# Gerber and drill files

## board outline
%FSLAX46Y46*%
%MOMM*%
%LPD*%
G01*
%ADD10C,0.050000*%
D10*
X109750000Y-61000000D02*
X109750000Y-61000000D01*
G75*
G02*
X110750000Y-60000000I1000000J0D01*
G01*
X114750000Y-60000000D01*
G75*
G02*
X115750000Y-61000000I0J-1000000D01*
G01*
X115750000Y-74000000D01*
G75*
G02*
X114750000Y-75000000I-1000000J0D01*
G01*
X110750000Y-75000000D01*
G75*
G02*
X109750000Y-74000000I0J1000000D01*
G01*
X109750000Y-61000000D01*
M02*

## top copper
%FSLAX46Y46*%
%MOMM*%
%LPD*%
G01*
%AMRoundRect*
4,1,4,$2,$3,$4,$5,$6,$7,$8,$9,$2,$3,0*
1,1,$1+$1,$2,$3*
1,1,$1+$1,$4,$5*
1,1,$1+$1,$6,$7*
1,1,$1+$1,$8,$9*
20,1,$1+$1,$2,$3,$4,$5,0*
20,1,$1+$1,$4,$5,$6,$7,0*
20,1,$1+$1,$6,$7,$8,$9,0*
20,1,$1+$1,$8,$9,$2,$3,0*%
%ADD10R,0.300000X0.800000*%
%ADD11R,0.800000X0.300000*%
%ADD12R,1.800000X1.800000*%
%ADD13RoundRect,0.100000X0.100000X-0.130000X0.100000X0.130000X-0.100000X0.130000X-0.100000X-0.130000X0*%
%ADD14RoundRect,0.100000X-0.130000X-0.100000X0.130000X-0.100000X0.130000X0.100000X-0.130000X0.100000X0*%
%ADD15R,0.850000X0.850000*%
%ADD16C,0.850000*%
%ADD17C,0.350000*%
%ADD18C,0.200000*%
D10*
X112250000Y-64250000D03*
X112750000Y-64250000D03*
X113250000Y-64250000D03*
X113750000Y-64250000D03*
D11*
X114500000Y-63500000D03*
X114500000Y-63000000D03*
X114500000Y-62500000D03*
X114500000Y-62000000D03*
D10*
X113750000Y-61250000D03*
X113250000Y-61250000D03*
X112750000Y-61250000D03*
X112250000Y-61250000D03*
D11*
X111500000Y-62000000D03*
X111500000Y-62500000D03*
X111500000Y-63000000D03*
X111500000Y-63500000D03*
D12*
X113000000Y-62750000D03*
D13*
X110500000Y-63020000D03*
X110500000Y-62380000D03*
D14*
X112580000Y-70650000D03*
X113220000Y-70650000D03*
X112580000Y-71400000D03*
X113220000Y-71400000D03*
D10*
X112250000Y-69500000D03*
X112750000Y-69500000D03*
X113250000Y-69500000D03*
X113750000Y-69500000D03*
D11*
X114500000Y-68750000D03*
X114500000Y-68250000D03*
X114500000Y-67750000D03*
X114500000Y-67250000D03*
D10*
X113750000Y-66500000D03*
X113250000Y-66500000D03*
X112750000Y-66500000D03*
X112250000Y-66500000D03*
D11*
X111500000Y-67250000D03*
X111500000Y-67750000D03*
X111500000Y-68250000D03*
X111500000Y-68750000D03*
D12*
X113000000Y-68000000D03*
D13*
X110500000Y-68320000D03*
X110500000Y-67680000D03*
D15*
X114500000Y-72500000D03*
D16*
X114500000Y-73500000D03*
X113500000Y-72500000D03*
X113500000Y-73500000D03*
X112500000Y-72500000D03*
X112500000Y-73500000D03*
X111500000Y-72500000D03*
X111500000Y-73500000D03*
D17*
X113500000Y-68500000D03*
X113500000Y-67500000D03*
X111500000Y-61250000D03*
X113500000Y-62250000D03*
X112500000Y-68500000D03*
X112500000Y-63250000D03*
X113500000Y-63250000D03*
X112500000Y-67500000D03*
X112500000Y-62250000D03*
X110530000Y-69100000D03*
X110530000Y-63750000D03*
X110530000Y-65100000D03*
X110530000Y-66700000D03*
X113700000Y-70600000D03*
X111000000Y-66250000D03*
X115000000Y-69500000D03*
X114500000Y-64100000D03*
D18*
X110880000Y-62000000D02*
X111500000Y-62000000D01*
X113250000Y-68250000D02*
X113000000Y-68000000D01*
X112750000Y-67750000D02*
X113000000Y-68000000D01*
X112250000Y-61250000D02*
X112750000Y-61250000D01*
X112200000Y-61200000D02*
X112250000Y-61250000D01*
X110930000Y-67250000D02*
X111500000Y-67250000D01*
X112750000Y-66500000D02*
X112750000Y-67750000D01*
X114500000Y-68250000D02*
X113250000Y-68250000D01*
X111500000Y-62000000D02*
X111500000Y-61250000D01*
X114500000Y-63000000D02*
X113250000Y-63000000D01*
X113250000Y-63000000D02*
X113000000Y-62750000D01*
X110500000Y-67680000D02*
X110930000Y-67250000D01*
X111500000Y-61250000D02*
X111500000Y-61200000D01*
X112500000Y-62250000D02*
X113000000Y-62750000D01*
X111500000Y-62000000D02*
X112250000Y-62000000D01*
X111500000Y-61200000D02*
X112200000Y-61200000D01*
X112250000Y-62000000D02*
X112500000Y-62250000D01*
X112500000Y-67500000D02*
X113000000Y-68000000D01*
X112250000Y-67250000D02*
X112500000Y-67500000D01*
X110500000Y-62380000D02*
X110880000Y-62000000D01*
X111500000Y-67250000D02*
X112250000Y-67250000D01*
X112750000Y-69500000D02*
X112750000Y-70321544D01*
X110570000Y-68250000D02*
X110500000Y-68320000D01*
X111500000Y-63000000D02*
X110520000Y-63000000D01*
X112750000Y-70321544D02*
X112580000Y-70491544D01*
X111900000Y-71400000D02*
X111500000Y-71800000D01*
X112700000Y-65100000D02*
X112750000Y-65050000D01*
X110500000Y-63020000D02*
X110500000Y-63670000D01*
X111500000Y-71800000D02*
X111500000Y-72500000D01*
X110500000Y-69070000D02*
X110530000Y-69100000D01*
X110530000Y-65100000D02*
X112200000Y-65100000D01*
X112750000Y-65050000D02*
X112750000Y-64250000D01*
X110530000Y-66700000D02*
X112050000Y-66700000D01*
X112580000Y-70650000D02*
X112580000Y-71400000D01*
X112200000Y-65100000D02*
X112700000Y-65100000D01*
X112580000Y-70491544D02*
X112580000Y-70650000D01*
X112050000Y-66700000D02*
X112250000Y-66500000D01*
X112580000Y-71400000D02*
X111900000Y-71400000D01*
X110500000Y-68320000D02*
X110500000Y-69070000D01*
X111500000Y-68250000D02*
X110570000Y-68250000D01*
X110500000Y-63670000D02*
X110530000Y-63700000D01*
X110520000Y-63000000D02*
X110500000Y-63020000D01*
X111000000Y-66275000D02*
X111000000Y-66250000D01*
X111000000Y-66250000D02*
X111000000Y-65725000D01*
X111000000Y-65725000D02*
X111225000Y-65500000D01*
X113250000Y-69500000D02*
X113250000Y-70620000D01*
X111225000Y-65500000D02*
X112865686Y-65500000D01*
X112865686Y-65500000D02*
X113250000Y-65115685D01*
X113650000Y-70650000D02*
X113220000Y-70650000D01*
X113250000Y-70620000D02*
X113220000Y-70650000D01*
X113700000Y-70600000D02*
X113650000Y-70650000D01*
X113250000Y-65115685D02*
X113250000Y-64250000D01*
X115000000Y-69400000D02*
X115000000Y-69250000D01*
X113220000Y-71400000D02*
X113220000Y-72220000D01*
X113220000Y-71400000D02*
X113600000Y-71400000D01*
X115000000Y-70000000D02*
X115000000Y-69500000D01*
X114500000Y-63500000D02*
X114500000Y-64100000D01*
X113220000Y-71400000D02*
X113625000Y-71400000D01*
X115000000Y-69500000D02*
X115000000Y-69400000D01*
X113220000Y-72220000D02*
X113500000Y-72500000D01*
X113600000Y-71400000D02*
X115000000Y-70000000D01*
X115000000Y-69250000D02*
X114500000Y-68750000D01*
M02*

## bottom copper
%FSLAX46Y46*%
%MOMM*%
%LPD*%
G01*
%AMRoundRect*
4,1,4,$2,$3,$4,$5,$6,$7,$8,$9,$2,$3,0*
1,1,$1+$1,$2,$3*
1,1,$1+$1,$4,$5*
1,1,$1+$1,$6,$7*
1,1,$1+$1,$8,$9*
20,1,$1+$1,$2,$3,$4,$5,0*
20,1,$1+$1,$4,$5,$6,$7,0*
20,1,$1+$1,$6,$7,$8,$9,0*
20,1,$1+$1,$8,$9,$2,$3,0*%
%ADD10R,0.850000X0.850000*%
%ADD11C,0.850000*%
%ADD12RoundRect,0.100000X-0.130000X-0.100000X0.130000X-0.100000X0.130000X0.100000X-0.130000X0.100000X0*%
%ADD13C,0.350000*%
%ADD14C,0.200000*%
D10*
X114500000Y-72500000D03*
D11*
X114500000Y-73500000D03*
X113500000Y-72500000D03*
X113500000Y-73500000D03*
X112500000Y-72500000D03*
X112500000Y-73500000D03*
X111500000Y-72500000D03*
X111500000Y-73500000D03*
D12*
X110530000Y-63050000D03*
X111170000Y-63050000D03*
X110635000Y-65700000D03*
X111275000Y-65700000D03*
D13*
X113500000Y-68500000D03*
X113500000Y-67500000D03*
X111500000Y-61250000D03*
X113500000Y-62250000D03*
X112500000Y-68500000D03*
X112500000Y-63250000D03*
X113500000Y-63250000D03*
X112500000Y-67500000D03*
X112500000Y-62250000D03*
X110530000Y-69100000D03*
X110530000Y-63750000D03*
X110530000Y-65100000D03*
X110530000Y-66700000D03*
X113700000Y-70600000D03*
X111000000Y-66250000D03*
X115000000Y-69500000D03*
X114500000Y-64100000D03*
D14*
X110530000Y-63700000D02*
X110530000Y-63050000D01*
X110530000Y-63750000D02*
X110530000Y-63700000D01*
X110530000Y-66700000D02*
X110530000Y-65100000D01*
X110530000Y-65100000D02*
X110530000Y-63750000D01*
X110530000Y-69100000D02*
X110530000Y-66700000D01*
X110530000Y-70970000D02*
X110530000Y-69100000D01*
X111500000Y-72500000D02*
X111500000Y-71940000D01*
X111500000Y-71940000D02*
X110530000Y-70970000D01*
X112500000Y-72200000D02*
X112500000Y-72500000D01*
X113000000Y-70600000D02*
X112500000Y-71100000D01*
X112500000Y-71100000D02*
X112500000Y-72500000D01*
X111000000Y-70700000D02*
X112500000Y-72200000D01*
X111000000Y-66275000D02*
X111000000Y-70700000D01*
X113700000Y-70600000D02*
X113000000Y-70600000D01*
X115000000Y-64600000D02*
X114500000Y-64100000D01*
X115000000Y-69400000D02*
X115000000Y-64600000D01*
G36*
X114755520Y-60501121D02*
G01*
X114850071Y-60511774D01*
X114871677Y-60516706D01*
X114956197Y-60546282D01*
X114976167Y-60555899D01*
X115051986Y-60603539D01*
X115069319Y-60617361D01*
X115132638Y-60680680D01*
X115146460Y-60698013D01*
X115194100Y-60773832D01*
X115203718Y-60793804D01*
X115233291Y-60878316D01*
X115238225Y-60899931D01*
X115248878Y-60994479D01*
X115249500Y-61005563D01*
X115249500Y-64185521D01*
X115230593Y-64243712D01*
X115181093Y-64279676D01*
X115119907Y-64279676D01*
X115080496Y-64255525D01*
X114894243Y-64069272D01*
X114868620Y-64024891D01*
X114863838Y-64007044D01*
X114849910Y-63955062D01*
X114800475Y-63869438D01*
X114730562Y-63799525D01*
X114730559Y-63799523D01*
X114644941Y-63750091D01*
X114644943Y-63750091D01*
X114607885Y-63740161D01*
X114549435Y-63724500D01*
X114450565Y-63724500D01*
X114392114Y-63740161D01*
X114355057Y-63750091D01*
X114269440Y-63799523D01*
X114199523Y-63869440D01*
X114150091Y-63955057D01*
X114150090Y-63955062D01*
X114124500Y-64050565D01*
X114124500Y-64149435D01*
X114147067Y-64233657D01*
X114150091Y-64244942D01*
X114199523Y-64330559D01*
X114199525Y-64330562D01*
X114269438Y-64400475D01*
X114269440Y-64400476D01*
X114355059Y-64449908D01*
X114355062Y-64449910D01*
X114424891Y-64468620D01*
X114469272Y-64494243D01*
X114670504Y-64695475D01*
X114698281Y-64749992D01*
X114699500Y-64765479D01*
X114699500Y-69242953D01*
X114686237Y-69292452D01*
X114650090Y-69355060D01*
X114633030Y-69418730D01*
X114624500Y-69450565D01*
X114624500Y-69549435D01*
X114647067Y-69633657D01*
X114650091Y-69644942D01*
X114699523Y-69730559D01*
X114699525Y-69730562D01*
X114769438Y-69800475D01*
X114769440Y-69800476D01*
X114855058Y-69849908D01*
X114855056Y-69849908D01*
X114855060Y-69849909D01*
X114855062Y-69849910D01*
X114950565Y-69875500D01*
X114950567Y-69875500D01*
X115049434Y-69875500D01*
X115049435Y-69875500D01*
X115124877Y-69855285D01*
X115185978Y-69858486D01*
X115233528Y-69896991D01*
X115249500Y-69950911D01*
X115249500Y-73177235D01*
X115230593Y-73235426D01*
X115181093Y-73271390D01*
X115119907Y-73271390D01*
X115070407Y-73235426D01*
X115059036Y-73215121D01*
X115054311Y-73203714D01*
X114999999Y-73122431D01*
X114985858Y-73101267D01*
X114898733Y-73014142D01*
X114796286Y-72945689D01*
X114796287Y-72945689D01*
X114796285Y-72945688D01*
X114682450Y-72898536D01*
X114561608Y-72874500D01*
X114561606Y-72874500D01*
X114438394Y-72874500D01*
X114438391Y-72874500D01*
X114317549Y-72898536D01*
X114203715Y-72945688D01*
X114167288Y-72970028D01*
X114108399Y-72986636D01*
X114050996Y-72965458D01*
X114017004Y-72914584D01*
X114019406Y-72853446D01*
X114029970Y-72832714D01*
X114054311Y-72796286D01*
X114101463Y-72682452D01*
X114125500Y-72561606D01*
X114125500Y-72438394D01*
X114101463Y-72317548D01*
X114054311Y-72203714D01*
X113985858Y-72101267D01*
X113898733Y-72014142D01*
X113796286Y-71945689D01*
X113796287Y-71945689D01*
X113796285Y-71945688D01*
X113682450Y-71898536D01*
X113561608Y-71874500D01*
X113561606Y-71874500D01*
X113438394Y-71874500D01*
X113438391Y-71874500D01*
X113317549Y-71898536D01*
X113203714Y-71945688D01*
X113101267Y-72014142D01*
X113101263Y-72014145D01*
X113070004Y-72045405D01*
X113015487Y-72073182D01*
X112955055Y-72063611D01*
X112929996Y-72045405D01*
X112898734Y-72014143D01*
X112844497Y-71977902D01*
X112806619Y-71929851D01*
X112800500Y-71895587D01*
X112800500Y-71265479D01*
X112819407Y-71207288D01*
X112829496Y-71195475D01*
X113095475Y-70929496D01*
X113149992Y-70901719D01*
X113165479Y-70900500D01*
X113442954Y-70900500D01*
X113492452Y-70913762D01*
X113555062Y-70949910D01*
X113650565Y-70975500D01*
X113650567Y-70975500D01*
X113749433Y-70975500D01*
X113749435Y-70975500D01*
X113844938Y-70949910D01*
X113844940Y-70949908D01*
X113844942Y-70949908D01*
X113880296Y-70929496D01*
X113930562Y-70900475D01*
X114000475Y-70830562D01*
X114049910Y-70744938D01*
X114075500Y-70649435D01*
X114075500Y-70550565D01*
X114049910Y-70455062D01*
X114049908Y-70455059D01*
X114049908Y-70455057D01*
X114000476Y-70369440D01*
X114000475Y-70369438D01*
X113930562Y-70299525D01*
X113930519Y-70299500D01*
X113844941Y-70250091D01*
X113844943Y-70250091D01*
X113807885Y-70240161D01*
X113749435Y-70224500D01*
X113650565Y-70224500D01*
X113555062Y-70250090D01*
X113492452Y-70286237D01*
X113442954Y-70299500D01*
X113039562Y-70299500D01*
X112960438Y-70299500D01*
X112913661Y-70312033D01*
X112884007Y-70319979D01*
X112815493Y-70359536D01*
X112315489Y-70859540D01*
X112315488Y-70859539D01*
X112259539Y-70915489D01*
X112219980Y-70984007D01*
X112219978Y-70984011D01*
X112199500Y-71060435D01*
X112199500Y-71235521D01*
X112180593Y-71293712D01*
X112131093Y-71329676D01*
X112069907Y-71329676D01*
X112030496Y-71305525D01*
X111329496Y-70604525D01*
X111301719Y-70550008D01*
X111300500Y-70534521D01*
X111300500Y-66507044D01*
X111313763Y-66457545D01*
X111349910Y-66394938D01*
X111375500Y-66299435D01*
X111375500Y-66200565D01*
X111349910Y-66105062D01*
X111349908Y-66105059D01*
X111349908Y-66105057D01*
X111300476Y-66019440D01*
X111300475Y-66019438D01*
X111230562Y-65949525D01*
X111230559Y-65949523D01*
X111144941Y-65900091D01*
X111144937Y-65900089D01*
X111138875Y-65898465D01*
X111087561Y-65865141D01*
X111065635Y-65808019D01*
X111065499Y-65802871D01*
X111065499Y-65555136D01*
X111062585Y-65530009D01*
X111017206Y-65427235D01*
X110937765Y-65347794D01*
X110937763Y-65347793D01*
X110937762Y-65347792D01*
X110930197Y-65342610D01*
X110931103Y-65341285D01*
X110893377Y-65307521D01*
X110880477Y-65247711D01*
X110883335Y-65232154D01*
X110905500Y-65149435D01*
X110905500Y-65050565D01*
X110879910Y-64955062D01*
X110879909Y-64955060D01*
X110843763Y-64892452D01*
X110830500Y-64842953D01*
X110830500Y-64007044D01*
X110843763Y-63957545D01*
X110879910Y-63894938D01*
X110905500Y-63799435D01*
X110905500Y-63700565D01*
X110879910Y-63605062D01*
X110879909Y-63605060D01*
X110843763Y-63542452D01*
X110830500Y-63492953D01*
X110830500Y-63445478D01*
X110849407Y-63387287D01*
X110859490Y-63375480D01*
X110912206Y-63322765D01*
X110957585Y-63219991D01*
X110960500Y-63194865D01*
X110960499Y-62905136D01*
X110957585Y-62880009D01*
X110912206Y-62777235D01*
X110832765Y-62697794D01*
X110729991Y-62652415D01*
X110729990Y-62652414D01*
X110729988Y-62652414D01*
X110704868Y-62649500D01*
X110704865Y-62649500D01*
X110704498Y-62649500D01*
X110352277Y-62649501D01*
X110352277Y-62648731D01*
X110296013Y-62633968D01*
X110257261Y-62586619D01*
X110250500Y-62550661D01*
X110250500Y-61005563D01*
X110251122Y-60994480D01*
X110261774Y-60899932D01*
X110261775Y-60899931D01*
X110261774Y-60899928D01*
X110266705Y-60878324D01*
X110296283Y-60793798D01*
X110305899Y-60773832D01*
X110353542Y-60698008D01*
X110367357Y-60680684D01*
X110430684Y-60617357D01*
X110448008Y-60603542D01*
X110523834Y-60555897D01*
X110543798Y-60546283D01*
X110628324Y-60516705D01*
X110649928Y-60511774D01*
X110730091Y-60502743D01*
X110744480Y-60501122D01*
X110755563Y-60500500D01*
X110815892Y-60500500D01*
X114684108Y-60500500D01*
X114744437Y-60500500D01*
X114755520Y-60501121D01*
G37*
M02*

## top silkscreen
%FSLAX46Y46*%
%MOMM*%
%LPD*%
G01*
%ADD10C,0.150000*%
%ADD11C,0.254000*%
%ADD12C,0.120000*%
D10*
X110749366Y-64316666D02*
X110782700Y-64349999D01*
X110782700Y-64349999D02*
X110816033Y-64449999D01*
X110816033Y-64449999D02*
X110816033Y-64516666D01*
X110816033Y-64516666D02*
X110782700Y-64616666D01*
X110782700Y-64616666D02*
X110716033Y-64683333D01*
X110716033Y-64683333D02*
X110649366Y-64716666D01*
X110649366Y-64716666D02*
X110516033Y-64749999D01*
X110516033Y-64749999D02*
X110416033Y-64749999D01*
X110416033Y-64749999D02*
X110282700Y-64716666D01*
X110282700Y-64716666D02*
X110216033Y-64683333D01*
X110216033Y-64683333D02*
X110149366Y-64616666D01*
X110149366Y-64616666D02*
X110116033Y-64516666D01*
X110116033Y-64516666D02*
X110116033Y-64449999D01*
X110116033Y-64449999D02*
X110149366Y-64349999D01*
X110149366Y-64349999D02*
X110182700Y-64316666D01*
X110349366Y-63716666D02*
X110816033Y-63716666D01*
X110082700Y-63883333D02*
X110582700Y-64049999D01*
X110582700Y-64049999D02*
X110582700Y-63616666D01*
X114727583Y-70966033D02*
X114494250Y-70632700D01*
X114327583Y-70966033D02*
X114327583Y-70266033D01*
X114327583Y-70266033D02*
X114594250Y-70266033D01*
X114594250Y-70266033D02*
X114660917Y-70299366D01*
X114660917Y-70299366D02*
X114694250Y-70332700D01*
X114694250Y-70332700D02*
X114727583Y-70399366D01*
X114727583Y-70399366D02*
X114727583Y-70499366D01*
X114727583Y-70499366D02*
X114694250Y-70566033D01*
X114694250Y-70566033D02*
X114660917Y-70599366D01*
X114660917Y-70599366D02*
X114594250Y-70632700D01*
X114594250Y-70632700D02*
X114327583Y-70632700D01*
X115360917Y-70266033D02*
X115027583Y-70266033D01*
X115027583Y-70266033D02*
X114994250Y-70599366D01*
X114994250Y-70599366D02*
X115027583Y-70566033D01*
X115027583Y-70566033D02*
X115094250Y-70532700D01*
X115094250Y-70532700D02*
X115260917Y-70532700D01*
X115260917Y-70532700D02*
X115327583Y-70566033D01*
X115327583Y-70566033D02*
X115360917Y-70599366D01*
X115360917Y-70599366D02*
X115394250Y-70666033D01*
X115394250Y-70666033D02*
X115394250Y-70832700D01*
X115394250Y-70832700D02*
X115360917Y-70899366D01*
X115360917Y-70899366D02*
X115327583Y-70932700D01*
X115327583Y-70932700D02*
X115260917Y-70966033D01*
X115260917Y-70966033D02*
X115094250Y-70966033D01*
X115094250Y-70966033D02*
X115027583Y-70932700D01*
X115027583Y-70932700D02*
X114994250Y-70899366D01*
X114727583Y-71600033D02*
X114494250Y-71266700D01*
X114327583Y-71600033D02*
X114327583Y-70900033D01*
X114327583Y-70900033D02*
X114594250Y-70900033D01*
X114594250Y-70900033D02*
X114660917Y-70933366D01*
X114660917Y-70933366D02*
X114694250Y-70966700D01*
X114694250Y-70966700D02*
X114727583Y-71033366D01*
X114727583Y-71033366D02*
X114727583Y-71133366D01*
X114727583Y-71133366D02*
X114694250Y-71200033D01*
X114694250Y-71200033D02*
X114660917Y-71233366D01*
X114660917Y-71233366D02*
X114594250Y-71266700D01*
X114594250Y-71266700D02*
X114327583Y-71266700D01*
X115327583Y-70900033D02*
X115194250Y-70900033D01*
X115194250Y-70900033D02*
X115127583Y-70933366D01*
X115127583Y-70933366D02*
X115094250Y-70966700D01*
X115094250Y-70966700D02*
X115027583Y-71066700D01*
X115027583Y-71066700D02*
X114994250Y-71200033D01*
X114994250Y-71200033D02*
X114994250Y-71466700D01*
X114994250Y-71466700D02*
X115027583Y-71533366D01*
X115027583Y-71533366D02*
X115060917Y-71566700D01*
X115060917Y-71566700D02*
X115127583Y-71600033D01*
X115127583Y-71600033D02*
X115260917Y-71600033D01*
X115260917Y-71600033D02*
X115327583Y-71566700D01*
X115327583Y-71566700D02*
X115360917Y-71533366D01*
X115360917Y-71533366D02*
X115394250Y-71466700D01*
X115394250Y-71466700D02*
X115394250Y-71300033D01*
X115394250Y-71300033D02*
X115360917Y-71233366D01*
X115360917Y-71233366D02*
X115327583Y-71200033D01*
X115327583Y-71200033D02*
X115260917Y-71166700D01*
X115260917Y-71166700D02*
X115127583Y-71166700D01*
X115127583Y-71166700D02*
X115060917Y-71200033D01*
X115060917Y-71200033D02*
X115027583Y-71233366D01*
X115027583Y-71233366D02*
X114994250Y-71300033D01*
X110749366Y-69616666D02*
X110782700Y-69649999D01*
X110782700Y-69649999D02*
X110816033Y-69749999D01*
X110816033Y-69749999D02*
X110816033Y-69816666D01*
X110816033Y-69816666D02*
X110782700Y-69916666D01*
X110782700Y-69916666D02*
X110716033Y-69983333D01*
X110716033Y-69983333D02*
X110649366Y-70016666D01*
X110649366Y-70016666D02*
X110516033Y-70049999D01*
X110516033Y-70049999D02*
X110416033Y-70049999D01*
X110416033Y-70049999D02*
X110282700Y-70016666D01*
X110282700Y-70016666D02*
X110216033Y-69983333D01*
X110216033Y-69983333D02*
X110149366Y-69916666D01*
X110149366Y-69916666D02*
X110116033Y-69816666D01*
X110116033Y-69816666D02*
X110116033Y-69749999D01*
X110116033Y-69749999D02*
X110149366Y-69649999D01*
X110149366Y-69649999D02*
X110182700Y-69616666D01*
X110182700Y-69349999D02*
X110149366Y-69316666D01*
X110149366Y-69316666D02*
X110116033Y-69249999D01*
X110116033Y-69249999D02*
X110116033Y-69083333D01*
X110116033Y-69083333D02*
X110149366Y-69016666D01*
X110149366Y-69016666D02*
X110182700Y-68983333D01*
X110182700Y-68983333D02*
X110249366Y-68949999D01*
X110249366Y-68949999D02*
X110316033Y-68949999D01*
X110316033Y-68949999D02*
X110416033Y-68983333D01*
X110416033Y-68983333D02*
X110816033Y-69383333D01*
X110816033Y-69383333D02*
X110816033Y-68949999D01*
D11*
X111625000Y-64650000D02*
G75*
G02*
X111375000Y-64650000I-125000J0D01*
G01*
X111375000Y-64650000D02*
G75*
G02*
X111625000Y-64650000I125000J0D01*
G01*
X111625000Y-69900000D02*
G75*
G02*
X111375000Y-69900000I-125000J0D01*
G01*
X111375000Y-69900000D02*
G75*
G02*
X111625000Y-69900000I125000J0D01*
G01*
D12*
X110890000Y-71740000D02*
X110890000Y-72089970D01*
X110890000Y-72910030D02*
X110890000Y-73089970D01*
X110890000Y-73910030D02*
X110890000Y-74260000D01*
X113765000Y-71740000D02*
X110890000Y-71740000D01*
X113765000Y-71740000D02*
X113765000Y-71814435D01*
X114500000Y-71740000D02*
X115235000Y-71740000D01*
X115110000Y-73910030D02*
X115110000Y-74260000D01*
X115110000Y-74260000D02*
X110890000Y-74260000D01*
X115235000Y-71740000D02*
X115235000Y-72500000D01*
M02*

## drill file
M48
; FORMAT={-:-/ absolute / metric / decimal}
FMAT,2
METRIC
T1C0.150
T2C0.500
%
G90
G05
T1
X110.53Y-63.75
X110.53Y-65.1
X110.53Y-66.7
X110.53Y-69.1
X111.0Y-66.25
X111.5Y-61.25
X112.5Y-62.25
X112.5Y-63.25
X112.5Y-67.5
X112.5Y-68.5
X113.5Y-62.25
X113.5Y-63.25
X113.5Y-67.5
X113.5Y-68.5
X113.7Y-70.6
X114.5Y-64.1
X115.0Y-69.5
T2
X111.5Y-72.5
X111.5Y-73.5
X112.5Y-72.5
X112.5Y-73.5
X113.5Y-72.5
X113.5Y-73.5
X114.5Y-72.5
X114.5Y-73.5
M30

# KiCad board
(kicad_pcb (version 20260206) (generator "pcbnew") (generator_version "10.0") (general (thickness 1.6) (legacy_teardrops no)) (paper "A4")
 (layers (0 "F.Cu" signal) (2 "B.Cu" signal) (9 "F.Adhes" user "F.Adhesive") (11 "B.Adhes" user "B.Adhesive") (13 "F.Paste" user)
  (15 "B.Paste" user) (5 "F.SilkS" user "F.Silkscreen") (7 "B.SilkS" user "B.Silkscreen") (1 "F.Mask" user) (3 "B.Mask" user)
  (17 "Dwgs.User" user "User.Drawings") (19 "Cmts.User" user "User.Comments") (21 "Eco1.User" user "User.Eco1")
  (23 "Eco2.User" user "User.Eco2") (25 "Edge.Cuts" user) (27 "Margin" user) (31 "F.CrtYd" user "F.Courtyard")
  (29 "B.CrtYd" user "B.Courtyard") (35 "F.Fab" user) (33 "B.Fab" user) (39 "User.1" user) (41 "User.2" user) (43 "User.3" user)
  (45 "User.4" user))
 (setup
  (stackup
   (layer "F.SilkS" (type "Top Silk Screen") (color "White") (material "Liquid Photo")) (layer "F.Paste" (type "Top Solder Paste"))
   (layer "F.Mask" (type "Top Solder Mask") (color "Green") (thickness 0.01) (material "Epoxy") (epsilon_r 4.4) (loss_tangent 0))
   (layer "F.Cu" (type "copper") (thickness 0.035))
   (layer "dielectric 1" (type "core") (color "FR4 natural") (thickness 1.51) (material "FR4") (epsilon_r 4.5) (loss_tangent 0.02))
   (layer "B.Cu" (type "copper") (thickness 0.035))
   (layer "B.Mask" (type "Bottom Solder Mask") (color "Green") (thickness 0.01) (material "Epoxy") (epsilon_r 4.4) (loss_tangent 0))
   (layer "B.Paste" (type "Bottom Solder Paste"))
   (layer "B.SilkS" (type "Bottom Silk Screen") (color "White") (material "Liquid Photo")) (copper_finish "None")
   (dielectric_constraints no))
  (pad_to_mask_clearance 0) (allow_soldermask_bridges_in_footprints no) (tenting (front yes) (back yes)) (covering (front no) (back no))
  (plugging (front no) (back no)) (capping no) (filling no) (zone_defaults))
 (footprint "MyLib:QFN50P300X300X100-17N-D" (layer "F.Cu") (at 113 62.75 90)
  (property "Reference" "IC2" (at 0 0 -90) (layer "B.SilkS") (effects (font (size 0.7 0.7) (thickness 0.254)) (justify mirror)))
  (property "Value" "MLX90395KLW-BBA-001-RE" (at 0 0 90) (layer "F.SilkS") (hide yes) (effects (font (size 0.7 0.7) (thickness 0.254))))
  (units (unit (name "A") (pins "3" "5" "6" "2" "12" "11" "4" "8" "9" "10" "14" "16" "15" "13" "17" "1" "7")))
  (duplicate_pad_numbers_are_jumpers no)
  (fp_circle (center -1.9 -1.5) (end -1.775 -1.5) (stroke (width 0.254) (type solid)) (fill no) (layer "F.SilkS"))
  (pad "1" smd rect (at -1.5 -0.75 180) (size 0.3 0.8) (layers "F.Cu" "F.Mask" "F.Paste") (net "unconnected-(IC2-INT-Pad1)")
   (thermal_bridge_angle 45))
  (pad "2" smd rect (at -1.5 -0.25 180) (size 0.3 0.8) (layers "F.Cu" "F.Mask" "F.Paste") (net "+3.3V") (thermal_bridge_angle 45))
  (pad "3" smd rect (at -1.5 0.25 180) (size 0.3 0.8) (layers "F.Cu" "F.Mask" "F.Paste") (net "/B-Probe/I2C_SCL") (thermal_bridge_angle 45))
  (pad "4" smd rect (at -1.5 0.75 180) (size 0.3 0.8) (layers "F.Cu" "F.Mask" "F.Paste") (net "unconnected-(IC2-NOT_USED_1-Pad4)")
   (thermal_bridge_angle 45))
  (pad "5" smd rect (at -0.75 1.5 90) (size 0.3 0.8) (layers "F.Cu" "F.Mask" "F.Paste") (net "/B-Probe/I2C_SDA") (thermal_bridge_angle 45))
  (pad "6" smd rect (at -0.25 1.5 90) (size 0.3 0.8) (layers "F.Cu" "F.Mask" "F.Paste") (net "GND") (thermal_bridge_angle 45))
  (pad "7" smd rect (at 0.25 1.5 90) (size 0.3 0.8) (layers "F.Cu" "F.Mask" "F.Paste") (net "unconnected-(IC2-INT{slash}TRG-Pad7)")
   (thermal_bridge_angle 45))
  (pad "8" smd rect (at 0.75 1.5 90) (size 0.3 0.8) (layers "F.Cu" "F.Mask" "F.Paste") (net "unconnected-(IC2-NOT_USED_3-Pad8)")
   (thermal_bridge_angle 45))
  (pad "9" smd rect (at 1.5 0.75 180) (size 0.3 0.8) (layers "F.Cu" "F.Mask" "F.Paste") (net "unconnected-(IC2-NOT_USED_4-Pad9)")
   (thermal_bridge_angle 45))
  (pad "10" smd rect (at 1.5 0.25 180) (size 0.3 0.8) (layers "F.Cu" "F.Mask" "F.Paste") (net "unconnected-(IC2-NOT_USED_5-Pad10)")
   (thermal_bridge_angle 45))
  (pad "11" smd rect (at 1.5 -0.25 180) (size 0.3 0.8) (layers "F.Cu" "F.Mask" "F.Paste") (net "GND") (thermal_bridge_angle 45))
  (pad "12" smd rect (at 1.5 -0.75 180) (size 0.3 0.8) (layers "F.Cu" "F.Mask" "F.Paste") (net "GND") (thermal_bridge_angle 45))
  (pad "13" smd rect (at 0.75 -1.5 90) (size 0.3 0.8) (layers "F.Cu" "F.Mask" "F.Paste") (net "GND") (thermal_bridge_angle 45))
  (pad "14" smd rect (at 0.25 -1.5 90) (size 0.3 0.8) (layers "F.Cu" "F.Mask" "F.Paste") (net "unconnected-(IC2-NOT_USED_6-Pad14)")
   (thermal_bridge_angle 45))
  (pad "15" smd rect (at -0.25 -1.5 90) (size 0.3 0.8) (layers "F.Cu" "F.Mask" "F.Paste") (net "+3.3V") (thermal_bridge_angle 45))
  (pad "16" smd rect (at -0.75 -1.5 90) (size 0.3 0.8) (layers "F.Cu" "F.Mask" "F.Paste") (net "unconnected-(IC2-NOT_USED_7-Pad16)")
   (thermal_bridge_angle 45))
  (pad "17" smd rect (at 0 0 90) (size 1.8 1.8) (layers "F.Cu" "F.Mask" "F.Paste") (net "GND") (thermal_bridge_angle 45)))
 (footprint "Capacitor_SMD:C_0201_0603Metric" (layer "F.Cu") (at 110.5 62.7 90)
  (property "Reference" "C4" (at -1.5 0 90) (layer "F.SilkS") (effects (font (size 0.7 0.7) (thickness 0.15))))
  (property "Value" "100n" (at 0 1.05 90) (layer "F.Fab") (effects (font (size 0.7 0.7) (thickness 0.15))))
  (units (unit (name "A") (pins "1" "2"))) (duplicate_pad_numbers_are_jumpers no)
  (pad "" smd roundrect (at -0.345 0 90) (size 0.318 0.36) (layers "F.Paste") (roundrect_rratio 0.25))
  (pad "" smd roundrect (at 0.345 0 90) (size 0.318 0.36) (layers "F.Paste") (roundrect_rratio 0.25))
  (pad "1" smd roundrect (at -0.32 0 90) (size 0.46 0.4) (layers "F.Cu" "F.Mask") (roundrect_rratio 0.25) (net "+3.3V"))
  (pad "2" smd roundrect (at 0.32 0 90) (size 0.46 0.4) (layers "F.Cu" "F.Mask") (roundrect_rratio 0.25) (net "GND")))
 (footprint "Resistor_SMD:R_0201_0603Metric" (layer "F.Cu") (at 112.9 70.65)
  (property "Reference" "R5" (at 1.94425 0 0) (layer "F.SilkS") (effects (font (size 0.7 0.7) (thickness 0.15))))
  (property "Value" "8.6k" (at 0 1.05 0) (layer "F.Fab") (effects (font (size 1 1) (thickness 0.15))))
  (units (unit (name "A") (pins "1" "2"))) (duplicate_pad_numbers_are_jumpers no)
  (pad "" smd roundrect (at -0.345 0) (size 0.318 0.36) (layers "F.Paste") (roundrect_rratio 0.25))
  (pad "" smd roundrect (at 0.345 0) (size 0.318 0.36) (layers "F.Paste") (roundrect_rratio 0.25))
  (pad "1" smd roundrect (at -0.32 0) (size 0.46 0.4) (layers "F.Cu" "F.Mask") (roundrect_rratio 0.25) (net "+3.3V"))
  (pad "2" smd roundrect (at 0.32 0) (size 0.46 0.4) (layers "F.Cu" "F.Mask") (roundrect_rratio 0.25) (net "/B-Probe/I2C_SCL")))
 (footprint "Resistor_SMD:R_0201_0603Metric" (layer "F.Cu") (at 112.9 71.4)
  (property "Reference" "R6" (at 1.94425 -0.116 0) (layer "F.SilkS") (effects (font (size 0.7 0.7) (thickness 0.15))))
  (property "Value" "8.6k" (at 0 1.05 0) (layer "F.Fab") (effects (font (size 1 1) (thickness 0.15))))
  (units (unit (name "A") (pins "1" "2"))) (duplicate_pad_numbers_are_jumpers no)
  (pad "" smd roundrect (at -0.345 0) (size 0.318 0.36) (layers "F.Paste") (roundrect_rratio 0.25))
  (pad "" smd roundrect (at 0.345 0) (size 0.318 0.36) (layers "F.Paste") (roundrect_rratio 0.25))
  (pad "1" smd roundrect (at -0.32 0) (size 0.46 0.4) (layers "F.Cu" "F.Mask") (roundrect_rratio 0.25) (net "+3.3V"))
  (pad "2" smd roundrect (at 0.32 0) (size 0.46 0.4) (layers "F.Cu" "F.Mask") (roundrect_rratio 0.25) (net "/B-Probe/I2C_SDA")))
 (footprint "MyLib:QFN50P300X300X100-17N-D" (layer "F.Cu") (at 113 68 90)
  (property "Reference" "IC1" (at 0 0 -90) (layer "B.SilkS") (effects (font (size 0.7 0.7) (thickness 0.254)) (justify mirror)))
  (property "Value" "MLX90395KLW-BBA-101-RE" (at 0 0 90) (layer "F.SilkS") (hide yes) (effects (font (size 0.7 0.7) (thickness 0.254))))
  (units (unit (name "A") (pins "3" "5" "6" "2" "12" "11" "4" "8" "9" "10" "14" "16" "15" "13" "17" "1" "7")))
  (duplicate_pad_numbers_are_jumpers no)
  (fp_circle (center -1.9 -1.5) (end -1.775 -1.5) (stroke (width 0.254) (type solid)) (fill no) (layer "F.SilkS"))
  (pad "1" smd rect (at -1.5 -0.75 180) (size 0.3 0.8) (layers "F.Cu" "F.Mask" "F.Paste") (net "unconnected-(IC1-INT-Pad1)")
   (thermal_bridge_angle 45))
  (pad "2" smd rect (at -1.5 -0.25 180) (size 0.3 0.8) (layers "F.Cu" "F.Mask" "F.Paste") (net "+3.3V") (thermal_bridge_angle 45))
  (pad "3" smd rect (at -1.5 0.25 180) (size 0.3 0.8) (layers "F.Cu" "F.Mask" "F.Paste") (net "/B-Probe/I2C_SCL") (thermal_bridge_angle 45))
  (pad "4" smd rect (at -1.5 0.75 180) (size 0.3 0.8) (layers "F.Cu" "F.Mask" "F.Paste") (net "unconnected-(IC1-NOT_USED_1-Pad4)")
   (thermal_bridge_angle 45))
  (pad "5" smd rect (at -0.75 1.5 90) (size 0.3 0.8) (layers "F.Cu" "F.Mask" "F.Paste") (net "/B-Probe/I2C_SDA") (thermal_bridge_angle 45))
  (pad "6" smd rect (at -0.25 1.5 90) (size 0.3 0.8) (layers "F.Cu" "F.Mask" "F.Paste") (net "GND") (thermal_bridge_angle 45))
  (pad "7" smd rect (at 0.25 1.5 90) (size 0.3 0.8) (layers "F.Cu" "F.Mask" "F.Paste") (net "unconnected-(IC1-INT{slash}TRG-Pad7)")
   (thermal_bridge_angle 45))
  (pad "8" smd rect (at 0.75 1.5 90) (size 0.3 0.8) (layers "F.Cu" "F.Mask" "F.Paste") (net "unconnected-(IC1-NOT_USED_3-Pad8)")
   (thermal_bridge_angle 45))
  (pad "9" smd rect (at 1.5 0.75 180) (size 0.3 0.8) (layers "F.Cu" "F.Mask" "F.Paste") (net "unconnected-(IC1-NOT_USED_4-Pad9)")
   (thermal_bridge_angle 45))
  (pad "10" smd rect (at 1.5 0.25 180) (size 0.3 0.8) (layers "F.Cu" "F.Mask" "F.Paste") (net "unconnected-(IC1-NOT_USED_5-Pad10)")
   (thermal_bridge_angle 45))
  (pad "11" smd rect (at 1.5 -0.25 180) (size 0.3 0.8) (layers "F.Cu" "F.Mask" "F.Paste") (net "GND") (thermal_bridge_angle 45))
  (pad "12" smd rect (at 1.5 -0.75 180) (size 0.3 0.8) (layers "F.Cu" "F.Mask" "F.Paste") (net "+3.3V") (thermal_bridge_angle 45))
  (pad "13" smd rect (at 0.75 -1.5 90) (size 0.3 0.8) (layers "F.Cu" "F.Mask" "F.Paste") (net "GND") (thermal_bridge_angle 45))
  (pad "14" smd rect (at 0.25 -1.5 90) (size 0.3 0.8) (layers "F.Cu" "F.Mask" "F.Paste") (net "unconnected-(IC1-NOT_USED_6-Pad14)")
   (thermal_bridge_angle 45))
  (pad "15" smd rect (at -0.25 -1.5 90) (size 0.3 0.8) (layers "F.Cu" "F.Mask" "F.Paste") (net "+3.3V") (thermal_bridge_angle 45))
  (pad "16" smd rect (at -0.75 -1.5 90) (size 0.3 0.8) (layers "F.Cu" "F.Mask" "F.Paste") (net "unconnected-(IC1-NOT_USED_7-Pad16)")
   (thermal_bridge_angle 45))
  (pad "17" smd rect (at 0 0 90) (size 1.8 1.8) (layers "F.Cu" "F.Mask" "F.Paste") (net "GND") (thermal_bridge_angle 45)))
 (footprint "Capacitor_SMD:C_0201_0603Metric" (layer "F.Cu") (at 110.5 68 90)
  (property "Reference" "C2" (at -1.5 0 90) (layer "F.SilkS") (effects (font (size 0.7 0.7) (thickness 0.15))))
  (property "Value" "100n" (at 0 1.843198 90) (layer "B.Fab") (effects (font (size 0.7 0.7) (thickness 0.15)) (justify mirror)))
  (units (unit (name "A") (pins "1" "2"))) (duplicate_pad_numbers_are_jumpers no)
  (pad "" smd roundrect (at -0.345 0 90) (size 0.318 0.36) (layers "F.Paste") (roundrect_rratio 0.25))
  (pad "" smd roundrect (at 0.345 0 90) (size 0.318 0.36) (layers "F.Paste") (roundrect_rratio 0.25))
  (pad "1" smd roundrect (at -0.32 0 90) (size 0.46 0.4) (layers "F.Cu" "F.Mask") (roundrect_rratio 0.25) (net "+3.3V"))
  (pad "2" smd roundrect (at 0.32 0 90) (size 0.46 0.4) (layers "F.Cu" "F.Mask") (roundrect_rratio 0.25) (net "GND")))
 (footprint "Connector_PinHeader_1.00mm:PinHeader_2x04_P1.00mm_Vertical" (layer "F.Cu") (at 114.5 72.5 -90)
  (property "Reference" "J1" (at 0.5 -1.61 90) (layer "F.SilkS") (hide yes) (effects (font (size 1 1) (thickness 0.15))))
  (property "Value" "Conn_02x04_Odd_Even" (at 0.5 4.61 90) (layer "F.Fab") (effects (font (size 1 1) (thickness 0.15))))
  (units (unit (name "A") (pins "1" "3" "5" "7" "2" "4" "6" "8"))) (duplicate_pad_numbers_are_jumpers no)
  (fp_line (start -0.76 3.61) (end -0.41003 3.61) (stroke (width 0.12) (type solid)) (layer "F.SilkS"))
  (fp_line (start 0.41003 3.61) (end 0.58997 3.61) (stroke (width 0.12) (type solid)) (layer "F.SilkS"))
  (fp_line (start 1.41003 3.61) (end 1.76 3.61) (stroke (width 0.12) (type solid)) (layer "F.SilkS"))
  (fp_line (start -0.76 0.735) (end -0.76 3.61) (stroke (width 0.12) (type solid)) (layer "F.SilkS"))
  (fp_line (start -0.76 0.735) (end -0.685565 0.735) (stroke (width 0.12) (type solid)) (layer "F.SilkS"))
  (fp_line (start -0.76 0) (end -0.76 -0.735) (stroke (width 0.12) (type solid)) (layer "F.SilkS"))
  (fp_line (start 1.41003 -0.61) (end 1.76 -0.61) (stroke (width 0.12) (type solid)) (layer "F.SilkS"))
  (fp_line (start 1.76 -0.61) (end 1.76 3.61) (stroke (width 0.12) (type solid)) (layer "F.SilkS"))
  (fp_line (start -0.76 -0.735) (end 0 -0.735) (stroke (width 0.12) (type solid)) (layer "F.SilkS"))
  (pad "1" thru_hole rect (at 0 0 270) (size 0.85 0.85) (drill 0.5) (layers "*.Cu" "*.Mask") (remove_unused_layers no) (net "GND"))
  (pad "2" thru_hole circle (at 1 0 270) (size 0.85 0.85) (drill 0.5) (layers "*.Cu" "*.Mask") (remove_unused_layers no)
   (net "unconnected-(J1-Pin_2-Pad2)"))
  (pad "3" thru_hole circle (at 0 1 270) (size 0.85 0.85) (drill 0.5) (layers "*.Cu" "*.Mask") (remove_unused_layers no)
   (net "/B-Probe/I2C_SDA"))
  (pad "4" thru_hole circle (at 1 1 270) (size 0.85 0.85) (drill 0.5) (layers "*.Cu" "*.Mask") (remove_unused_layers no)
   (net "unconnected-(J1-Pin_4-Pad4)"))
  (pad "5" thru_hole circle (at 0 2 270) (size 0.85 0.85) (drill 0.5) (layers "*.Cu" "*.Mask") (remove_unused_layers no)
   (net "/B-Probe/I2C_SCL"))
  (pad "6" thru_hole circle (at 1 2 270) (size 0.85 0.85) (drill 0.5) (layers "*.Cu" "*.Mask") (remove_unused_layers no)
   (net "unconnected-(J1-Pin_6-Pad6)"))
  (pad "7" thru_hole circle (at 0 3 270) (size 0.85 0.85) (drill 0.5) (layers "*.Cu" "*.Mask") (remove_unused_layers no) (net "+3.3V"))
  (pad "8" thru_hole circle (at 1 3 270) (size 0.85 0.85) (drill 0.5) (layers "*.Cu" "*.Mask") (remove_unused_layers no)
   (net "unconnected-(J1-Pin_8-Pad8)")))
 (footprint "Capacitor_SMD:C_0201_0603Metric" (layer "B.Cu") (at 110.85 63.05)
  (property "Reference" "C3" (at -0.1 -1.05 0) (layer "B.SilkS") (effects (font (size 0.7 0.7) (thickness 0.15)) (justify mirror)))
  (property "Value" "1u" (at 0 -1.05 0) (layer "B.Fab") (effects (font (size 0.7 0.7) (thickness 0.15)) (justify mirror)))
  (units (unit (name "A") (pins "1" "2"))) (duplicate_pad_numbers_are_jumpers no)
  (pad "" smd roundrect (at -0.345 0) (size 0.318 0.36) (layers "B.Paste") (roundrect_rratio 0.25))
  (pad "" smd roundrect (at 0.345 0) (size 0.318 0.36) (layers "B.Paste") (roundrect_rratio 0.25))
  (pad "1" smd roundrect (at -0.32 0) (size 0.46 0.4) (layers "B.Cu" "B.Mask") (roundrect_rratio 0.25) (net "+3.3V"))
  (pad "2" smd roundrect (at 0.32 0) (size 0.46 0.4) (layers "B.Cu" "B.Mask") (roundrect_rratio 0.25) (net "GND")))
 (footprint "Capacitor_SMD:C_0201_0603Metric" (layer "B.Cu") (at 110.955 65.7)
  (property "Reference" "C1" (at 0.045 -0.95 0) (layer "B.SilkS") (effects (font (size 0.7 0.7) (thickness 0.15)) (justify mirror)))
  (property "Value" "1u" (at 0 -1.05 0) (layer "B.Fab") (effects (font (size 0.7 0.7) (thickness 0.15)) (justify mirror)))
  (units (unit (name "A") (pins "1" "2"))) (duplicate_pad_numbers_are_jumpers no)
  (pad "" smd roundrect (at -0.345 0) (size 0.318 0.36) (layers "B.Paste") (roundrect_rratio 0.25))
  (pad "" smd roundrect (at 0.345 0) (size 0.318 0.36) (layers "B.Paste") (roundrect_rratio 0.25))
  (pad "1" smd roundrect (at -0.32 0) (size 0.46 0.4) (layers "B.Cu" "B.Mask") (roundrect_rratio 0.25) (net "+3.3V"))
  (pad "2" smd roundrect (at 0.32 0) (size 0.46 0.4) (layers "B.Cu" "B.Mask") (roundrect_rratio 0.25) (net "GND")))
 (gr_rect (start 109.75 60) (end 115.75 75) (radius 1) (stroke (width 0.05) (type solid)) (fill no) (layer "Edge.Cuts"))
 (segment (start 110.88 62) (end 111.5 62) (width 0.2) (layer "F.Cu") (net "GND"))
 (segment (start 113.25 68.25) (end 113 68) (width 0.2) (layer "F.Cu") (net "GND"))
 (segment (start 112.75 67.75) (end 113 68) (width 0.2) (layer "F.Cu") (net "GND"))
 (segment (start 112.25 61.25) (end 112.75 61.25) (width 0.2) (layer "F.Cu") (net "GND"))
 (segment (start 112.2 61.2) (end 112.25 61.25) (width 0.2) (layer "F.Cu") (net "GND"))
 (segment (start 110.93 67.25) (end 111.5 67.25) (width 0.2) (layer "F.Cu") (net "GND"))
 (segment (start 112.75 66.5) (end 112.75 67.75) (width 0.2) (layer "F.Cu") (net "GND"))
 (segment (start 114.5 68.25) (end 113.25 68.25) (width 0.2) (layer "F.Cu") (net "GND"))
 (segment (start 111.5 62) (end 111.5 61.25) (width 0.2) (layer "F.Cu") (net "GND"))
 (segment (start 114.5 63) (end 113.25 63) (width 0.2) (layer "F.Cu") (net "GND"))
 (segment (start 113.25 63) (end 113 62.75) (width 0.2) (layer "F.Cu") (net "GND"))
 (segment (start 110.5 67.68) (end 110.93 67.25) (width 0.2) (layer "F.Cu") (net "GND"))
 (segment (start 111.5 61.25) (end 111.5 61.2) (width 0.2) (layer "F.Cu") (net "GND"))
 (segment (start 112.5 62.25) (end 113 62.75) (width 0.2) (layer "F.Cu") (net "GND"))
 (segment (start 111.5 62) (end 112.25 62) (width 0.2) (layer "F.Cu") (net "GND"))
 (segment (start 111.5 61.2) (end 112.2 61.2) (width 0.2) (layer "F.Cu") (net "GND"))
 (segment (start 112.25 62) (end 112.5 62.25) (width 0.2) (layer "F.Cu") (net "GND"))
 (segment (start 112.5 67.5) (end 113 68) (width 0.2) (layer "F.Cu") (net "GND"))
 (segment (start 112.25 67.25) (end 112.5 67.5) (width 0.2) (layer "F.Cu") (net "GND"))
 (segment (start 110.5 62.38) (end 110.88 62) (width 0.2) (layer "F.Cu") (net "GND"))
 (segment (start 111.5 67.25) (end 112.25 67.25) (width 0.2) (layer "F.Cu") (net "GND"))
 (via (at 113.5 68.5) (size 0.35) (drill 0.15) (layers "F.Cu" "B.Cu") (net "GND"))
 (via (at 113.5 67.5) (size 0.35) (drill 0.15) (layers "F.Cu" "B.Cu") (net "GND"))
 (via (at 111.5 61.25) (size 0.35) (drill 0.15) (layers "F.Cu" "B.Cu") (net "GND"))
 (via (at 113.5 62.25) (size 0.35) (drill 0.15) (layers "F.Cu" "B.Cu") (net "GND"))
 (via (at 112.5 68.5) (size 0.35) (drill 0.15) (layers "F.Cu" "B.Cu") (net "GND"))
 (via (at 112.5 63.25) (size 0.35) (drill 0.15) (layers "F.Cu" "B.Cu") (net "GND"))
 (via (at 113.5 63.25) (size 0.35) (drill 0.15) (layers "F.Cu" "B.Cu") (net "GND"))
 (via (at 112.5 67.5) (size 0.35) (drill 0.15) (layers "F.Cu" "B.Cu") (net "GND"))
 (via (at 112.5 62.25) (size 0.35) (drill 0.15) (layers "F.Cu" "B.Cu") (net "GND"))
 (segment (start 112.75 69.5) (end 112.75 70.321544) (width 0.2) (layer "F.Cu") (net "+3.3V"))
 (segment (start 110.57 68.25) (end 110.5 68.32) (width 0.2) (layer "F.Cu") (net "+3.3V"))
 (segment (start 111.5 63) (end 110.52 63) (width 0.2) (layer "F.Cu") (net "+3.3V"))
 (segment (start 112.75 70.321544) (end 112.58 70.491544) (width 0.2) (layer "F.Cu") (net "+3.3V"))
 (segment (start 111.9 71.4) (end 111.5 71.8) (width 0.2) (layer "F.Cu") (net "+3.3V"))
 (segment (start 112.7 65.1) (end 112.75 65.05) (width 0.2) (layer "F.Cu") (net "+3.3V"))
 (segment (start 110.5 63.02) (end 110.5 63.67) (width 0.2) (layer "F.Cu") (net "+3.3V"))
 (segment (start 111.5 71.8) (end 111.5 72.5) (width 0.2) (layer "F.Cu") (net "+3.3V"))
 (segment (start 110.5 69.07) (end 110.53 69.1) (width 0.2) (layer "F.Cu") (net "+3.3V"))
 (segment (start 110.53 65.1) (end 112.2 65.1) (width 0.2) (layer "F.Cu") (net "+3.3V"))
 (segment (start 112.75 65.05) (end 112.75 64.25) (width 0.2) (layer "F.Cu") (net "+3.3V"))
 (segment (start 110.53 66.7) (end 112.05 66.7) (width 0.2) (layer "F.Cu") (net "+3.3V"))
 (segment (start 112.58 70.65) (end 112.58 71.4) (width 0.2) (layer "F.Cu") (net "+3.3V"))
 (segment (start 112.2 65.1) (end 112.7 65.1) (width 0.2) (layer "F.Cu") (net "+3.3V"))
 (segment (start 112.58 70.491544) (end 112.58 70.65) (width 0.2) (layer "F.Cu") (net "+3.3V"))
 (segment (start 112.05 66.7) (end 112.25 66.5) (width 0.2) (layer "F.Cu") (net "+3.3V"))
 (segment (start 112.58 71.4) (end 111.9 71.4) (width 0.2) (layer "F.Cu") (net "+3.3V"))
 (segment (start 110.5 68.32) (end 110.5 69.07) (width 0.2) (layer "F.Cu") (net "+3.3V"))
 (segment (start 111.5 68.25) (end 110.57 68.25) (width 0.2) (layer "F.Cu") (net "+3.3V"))
 (segment (start 110.5 63.67) (end 110.53 63.7) (width 0.2) (layer "F.Cu") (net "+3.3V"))
 (segment (start 110.52 63) (end 110.5 63.02) (width 0.2) (layer "F.Cu") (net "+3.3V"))
 (via (at 110.53 69.1) (size 0.35) (drill 0.15) (layers "F.Cu" "B.Cu") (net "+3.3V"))
 (via (at 110.53 63.75) (size 0.35) (drill 0.15) (layers "F.Cu" "B.Cu") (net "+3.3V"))
 (via (at 110.53 65.1) (size 0.35) (drill 0.15) (layers "F.Cu" "B.Cu") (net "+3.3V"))
 (via (at 110.53 66.7) (size 0.35) (drill 0.15) (layers "F.Cu" "B.Cu") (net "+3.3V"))
 (segment (start 110.53 63.7) (end 110.53 63.05) (width 0.2) (layer "B.Cu") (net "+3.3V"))
 (segment (start 110.53 63.75) (end 110.53 63.7) (width 0.2) (layer "B.Cu") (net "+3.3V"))
 (segment (start 110.53 66.7) (end 110.53 65.1) (width 0.2) (layer "B.Cu") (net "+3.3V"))
 (segment (start 110.53 65.1) (end 110.53 63.75) (width 0.2) (layer "B.Cu") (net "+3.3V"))
 (segment (start 110.53 69.1) (end 110.53 66.7) (width 0.2) (layer "B.Cu") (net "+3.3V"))
 (segment (start 110.53 70.97) (end 110.53 69.1) (width 0.2) (layer "B.Cu") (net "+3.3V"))
 (segment (start 111.5 72.5) (end 111.5 71.94) (width 0.2) (layer "B.Cu") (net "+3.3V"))
 (segment (start 111.5 71.94) (end 110.53 70.97) (width 0.2) (layer "B.Cu") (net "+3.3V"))
 (segment (start 111 66.275) (end 111 66.25) (width 0.2) (layer "F.Cu") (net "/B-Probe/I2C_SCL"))
 (segment (start 111 66.25) (end 111 65.725) (width 0.2) (layer "F.Cu") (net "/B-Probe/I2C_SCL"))
 (segment (start 111 65.725) (end 111.225 65.5) (width 0.2) (layer "F.Cu") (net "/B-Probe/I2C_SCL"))
 (segment (start 113.25 69.5) (end 113.25 70.62) (width 0.2) (layer "F.Cu") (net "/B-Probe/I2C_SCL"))
 (segment (start 111.225 65.5) (end 112.865686 65.5) (width 0.2) (layer "F.Cu") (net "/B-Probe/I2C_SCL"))
 (segment (start 112.865686 65.5) (end 113.25 65.115685) (width 0.2) (layer "F.Cu") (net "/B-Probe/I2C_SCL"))
 (segment (start 113.65 70.65) (end 113.22 70.65) (width 0.2) (layer "F.Cu") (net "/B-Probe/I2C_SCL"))
 (segment (start 113.25 70.62) (end 113.22 70.65) (width 0.2) (layer "F.Cu") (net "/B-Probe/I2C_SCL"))
 (segment (start 113.7 70.6) (end 113.65 70.65) (width 0.2) (layer "F.Cu") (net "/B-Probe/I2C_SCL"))
 (segment (start 113.25 65.115685) (end 113.25 64.25) (width 0.2) (layer "F.Cu") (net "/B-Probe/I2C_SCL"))
 (via (at 113.7 70.6) (size 0.35) (drill 0.15) (layers "F.Cu" "B.Cu") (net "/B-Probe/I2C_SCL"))
 (via (at 111 66.25) (size 0.35) (drill 0.15) (layers "F.Cu" "B.Cu") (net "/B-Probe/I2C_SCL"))
 (segment (start 112.5 72.2) (end 112.5 72.5) (width 0.2) (layer "B.Cu") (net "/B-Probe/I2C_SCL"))
 (segment (start 113 70.6) (end 112.5 71.1) (width 0.2) (layer "B.Cu") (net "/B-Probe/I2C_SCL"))
 (segment (start 112.5 71.1) (end 112.5 72.5) (width 0.2) (layer "B.Cu") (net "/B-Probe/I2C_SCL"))
 (segment (start 111 70.7) (end 112.5 72.2) (width 0.2) (layer "B.Cu") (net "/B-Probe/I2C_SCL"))
 (segment (start 111 66.275) (end 111 70.7) (width 0.2) (layer "B.Cu") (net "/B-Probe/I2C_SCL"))
 (segment (start 113.7 70.6) (end 113 70.6) (width 0.2) (layer "B.Cu") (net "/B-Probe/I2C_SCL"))
 (segment (start 115 69.4) (end 115 69.25) (width 0.2) (layer "F.Cu") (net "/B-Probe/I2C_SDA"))
 (segment (start 113.22 71.4) (end 113.22 72.22) (width 0.2) (layer "F.Cu") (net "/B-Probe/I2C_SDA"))
 (segment (start 113.22 71.4) (end 113.6 71.4) (width 0.2) (layer "F.Cu") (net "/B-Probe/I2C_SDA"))
 (segment (start 115 70) (end 115 69.5) (width 0.2) (layer "F.Cu") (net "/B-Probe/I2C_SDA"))
 (segment (start 114.5 63.5) (end 114.5 64.1) (width 0.2) (layer "F.Cu") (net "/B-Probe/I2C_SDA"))
 (segment (start 113.22 71.4) (end 113.625 71.4) (width 0.2) (layer "F.Cu") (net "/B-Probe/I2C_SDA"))
 (segment (start 115 69.5) (end 115 69.4) (width 0.2) (layer "F.Cu") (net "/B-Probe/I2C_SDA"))
 (segment (start 113.22 72.22) (end 113.5 72.5) (width 0.2) (layer "F.Cu") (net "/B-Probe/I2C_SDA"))
 (segment (start 113.6 71.4) (end 115 70) (width 0.2) (layer "F.Cu") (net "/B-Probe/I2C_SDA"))
 (segment (start 115 69.25) (end 114.5 68.75) (width 0.2) (layer "F.Cu") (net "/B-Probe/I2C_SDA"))
 (via (at 115 69.5) (size 0.35) (drill 0.15) (layers "F.Cu" "B.Cu") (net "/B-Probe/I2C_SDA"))
 (via (at 114.5 64.1) (size 0.35) (drill 0.15) (layers "F.Cu" "B.Cu") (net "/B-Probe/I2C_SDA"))
 (segment (start 115 64.6) (end 114.5 64.1) (width 0.2) (layer "B.Cu") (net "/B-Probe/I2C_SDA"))
 (segment (start 115 69.4) (end 115 64.6) (width 0.2) (layer "B.Cu") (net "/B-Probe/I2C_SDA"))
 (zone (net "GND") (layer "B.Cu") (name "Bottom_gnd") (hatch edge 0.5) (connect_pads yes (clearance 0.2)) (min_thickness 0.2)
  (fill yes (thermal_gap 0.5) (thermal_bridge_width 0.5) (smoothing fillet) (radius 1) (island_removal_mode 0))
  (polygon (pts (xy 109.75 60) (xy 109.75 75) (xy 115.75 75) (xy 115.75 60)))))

